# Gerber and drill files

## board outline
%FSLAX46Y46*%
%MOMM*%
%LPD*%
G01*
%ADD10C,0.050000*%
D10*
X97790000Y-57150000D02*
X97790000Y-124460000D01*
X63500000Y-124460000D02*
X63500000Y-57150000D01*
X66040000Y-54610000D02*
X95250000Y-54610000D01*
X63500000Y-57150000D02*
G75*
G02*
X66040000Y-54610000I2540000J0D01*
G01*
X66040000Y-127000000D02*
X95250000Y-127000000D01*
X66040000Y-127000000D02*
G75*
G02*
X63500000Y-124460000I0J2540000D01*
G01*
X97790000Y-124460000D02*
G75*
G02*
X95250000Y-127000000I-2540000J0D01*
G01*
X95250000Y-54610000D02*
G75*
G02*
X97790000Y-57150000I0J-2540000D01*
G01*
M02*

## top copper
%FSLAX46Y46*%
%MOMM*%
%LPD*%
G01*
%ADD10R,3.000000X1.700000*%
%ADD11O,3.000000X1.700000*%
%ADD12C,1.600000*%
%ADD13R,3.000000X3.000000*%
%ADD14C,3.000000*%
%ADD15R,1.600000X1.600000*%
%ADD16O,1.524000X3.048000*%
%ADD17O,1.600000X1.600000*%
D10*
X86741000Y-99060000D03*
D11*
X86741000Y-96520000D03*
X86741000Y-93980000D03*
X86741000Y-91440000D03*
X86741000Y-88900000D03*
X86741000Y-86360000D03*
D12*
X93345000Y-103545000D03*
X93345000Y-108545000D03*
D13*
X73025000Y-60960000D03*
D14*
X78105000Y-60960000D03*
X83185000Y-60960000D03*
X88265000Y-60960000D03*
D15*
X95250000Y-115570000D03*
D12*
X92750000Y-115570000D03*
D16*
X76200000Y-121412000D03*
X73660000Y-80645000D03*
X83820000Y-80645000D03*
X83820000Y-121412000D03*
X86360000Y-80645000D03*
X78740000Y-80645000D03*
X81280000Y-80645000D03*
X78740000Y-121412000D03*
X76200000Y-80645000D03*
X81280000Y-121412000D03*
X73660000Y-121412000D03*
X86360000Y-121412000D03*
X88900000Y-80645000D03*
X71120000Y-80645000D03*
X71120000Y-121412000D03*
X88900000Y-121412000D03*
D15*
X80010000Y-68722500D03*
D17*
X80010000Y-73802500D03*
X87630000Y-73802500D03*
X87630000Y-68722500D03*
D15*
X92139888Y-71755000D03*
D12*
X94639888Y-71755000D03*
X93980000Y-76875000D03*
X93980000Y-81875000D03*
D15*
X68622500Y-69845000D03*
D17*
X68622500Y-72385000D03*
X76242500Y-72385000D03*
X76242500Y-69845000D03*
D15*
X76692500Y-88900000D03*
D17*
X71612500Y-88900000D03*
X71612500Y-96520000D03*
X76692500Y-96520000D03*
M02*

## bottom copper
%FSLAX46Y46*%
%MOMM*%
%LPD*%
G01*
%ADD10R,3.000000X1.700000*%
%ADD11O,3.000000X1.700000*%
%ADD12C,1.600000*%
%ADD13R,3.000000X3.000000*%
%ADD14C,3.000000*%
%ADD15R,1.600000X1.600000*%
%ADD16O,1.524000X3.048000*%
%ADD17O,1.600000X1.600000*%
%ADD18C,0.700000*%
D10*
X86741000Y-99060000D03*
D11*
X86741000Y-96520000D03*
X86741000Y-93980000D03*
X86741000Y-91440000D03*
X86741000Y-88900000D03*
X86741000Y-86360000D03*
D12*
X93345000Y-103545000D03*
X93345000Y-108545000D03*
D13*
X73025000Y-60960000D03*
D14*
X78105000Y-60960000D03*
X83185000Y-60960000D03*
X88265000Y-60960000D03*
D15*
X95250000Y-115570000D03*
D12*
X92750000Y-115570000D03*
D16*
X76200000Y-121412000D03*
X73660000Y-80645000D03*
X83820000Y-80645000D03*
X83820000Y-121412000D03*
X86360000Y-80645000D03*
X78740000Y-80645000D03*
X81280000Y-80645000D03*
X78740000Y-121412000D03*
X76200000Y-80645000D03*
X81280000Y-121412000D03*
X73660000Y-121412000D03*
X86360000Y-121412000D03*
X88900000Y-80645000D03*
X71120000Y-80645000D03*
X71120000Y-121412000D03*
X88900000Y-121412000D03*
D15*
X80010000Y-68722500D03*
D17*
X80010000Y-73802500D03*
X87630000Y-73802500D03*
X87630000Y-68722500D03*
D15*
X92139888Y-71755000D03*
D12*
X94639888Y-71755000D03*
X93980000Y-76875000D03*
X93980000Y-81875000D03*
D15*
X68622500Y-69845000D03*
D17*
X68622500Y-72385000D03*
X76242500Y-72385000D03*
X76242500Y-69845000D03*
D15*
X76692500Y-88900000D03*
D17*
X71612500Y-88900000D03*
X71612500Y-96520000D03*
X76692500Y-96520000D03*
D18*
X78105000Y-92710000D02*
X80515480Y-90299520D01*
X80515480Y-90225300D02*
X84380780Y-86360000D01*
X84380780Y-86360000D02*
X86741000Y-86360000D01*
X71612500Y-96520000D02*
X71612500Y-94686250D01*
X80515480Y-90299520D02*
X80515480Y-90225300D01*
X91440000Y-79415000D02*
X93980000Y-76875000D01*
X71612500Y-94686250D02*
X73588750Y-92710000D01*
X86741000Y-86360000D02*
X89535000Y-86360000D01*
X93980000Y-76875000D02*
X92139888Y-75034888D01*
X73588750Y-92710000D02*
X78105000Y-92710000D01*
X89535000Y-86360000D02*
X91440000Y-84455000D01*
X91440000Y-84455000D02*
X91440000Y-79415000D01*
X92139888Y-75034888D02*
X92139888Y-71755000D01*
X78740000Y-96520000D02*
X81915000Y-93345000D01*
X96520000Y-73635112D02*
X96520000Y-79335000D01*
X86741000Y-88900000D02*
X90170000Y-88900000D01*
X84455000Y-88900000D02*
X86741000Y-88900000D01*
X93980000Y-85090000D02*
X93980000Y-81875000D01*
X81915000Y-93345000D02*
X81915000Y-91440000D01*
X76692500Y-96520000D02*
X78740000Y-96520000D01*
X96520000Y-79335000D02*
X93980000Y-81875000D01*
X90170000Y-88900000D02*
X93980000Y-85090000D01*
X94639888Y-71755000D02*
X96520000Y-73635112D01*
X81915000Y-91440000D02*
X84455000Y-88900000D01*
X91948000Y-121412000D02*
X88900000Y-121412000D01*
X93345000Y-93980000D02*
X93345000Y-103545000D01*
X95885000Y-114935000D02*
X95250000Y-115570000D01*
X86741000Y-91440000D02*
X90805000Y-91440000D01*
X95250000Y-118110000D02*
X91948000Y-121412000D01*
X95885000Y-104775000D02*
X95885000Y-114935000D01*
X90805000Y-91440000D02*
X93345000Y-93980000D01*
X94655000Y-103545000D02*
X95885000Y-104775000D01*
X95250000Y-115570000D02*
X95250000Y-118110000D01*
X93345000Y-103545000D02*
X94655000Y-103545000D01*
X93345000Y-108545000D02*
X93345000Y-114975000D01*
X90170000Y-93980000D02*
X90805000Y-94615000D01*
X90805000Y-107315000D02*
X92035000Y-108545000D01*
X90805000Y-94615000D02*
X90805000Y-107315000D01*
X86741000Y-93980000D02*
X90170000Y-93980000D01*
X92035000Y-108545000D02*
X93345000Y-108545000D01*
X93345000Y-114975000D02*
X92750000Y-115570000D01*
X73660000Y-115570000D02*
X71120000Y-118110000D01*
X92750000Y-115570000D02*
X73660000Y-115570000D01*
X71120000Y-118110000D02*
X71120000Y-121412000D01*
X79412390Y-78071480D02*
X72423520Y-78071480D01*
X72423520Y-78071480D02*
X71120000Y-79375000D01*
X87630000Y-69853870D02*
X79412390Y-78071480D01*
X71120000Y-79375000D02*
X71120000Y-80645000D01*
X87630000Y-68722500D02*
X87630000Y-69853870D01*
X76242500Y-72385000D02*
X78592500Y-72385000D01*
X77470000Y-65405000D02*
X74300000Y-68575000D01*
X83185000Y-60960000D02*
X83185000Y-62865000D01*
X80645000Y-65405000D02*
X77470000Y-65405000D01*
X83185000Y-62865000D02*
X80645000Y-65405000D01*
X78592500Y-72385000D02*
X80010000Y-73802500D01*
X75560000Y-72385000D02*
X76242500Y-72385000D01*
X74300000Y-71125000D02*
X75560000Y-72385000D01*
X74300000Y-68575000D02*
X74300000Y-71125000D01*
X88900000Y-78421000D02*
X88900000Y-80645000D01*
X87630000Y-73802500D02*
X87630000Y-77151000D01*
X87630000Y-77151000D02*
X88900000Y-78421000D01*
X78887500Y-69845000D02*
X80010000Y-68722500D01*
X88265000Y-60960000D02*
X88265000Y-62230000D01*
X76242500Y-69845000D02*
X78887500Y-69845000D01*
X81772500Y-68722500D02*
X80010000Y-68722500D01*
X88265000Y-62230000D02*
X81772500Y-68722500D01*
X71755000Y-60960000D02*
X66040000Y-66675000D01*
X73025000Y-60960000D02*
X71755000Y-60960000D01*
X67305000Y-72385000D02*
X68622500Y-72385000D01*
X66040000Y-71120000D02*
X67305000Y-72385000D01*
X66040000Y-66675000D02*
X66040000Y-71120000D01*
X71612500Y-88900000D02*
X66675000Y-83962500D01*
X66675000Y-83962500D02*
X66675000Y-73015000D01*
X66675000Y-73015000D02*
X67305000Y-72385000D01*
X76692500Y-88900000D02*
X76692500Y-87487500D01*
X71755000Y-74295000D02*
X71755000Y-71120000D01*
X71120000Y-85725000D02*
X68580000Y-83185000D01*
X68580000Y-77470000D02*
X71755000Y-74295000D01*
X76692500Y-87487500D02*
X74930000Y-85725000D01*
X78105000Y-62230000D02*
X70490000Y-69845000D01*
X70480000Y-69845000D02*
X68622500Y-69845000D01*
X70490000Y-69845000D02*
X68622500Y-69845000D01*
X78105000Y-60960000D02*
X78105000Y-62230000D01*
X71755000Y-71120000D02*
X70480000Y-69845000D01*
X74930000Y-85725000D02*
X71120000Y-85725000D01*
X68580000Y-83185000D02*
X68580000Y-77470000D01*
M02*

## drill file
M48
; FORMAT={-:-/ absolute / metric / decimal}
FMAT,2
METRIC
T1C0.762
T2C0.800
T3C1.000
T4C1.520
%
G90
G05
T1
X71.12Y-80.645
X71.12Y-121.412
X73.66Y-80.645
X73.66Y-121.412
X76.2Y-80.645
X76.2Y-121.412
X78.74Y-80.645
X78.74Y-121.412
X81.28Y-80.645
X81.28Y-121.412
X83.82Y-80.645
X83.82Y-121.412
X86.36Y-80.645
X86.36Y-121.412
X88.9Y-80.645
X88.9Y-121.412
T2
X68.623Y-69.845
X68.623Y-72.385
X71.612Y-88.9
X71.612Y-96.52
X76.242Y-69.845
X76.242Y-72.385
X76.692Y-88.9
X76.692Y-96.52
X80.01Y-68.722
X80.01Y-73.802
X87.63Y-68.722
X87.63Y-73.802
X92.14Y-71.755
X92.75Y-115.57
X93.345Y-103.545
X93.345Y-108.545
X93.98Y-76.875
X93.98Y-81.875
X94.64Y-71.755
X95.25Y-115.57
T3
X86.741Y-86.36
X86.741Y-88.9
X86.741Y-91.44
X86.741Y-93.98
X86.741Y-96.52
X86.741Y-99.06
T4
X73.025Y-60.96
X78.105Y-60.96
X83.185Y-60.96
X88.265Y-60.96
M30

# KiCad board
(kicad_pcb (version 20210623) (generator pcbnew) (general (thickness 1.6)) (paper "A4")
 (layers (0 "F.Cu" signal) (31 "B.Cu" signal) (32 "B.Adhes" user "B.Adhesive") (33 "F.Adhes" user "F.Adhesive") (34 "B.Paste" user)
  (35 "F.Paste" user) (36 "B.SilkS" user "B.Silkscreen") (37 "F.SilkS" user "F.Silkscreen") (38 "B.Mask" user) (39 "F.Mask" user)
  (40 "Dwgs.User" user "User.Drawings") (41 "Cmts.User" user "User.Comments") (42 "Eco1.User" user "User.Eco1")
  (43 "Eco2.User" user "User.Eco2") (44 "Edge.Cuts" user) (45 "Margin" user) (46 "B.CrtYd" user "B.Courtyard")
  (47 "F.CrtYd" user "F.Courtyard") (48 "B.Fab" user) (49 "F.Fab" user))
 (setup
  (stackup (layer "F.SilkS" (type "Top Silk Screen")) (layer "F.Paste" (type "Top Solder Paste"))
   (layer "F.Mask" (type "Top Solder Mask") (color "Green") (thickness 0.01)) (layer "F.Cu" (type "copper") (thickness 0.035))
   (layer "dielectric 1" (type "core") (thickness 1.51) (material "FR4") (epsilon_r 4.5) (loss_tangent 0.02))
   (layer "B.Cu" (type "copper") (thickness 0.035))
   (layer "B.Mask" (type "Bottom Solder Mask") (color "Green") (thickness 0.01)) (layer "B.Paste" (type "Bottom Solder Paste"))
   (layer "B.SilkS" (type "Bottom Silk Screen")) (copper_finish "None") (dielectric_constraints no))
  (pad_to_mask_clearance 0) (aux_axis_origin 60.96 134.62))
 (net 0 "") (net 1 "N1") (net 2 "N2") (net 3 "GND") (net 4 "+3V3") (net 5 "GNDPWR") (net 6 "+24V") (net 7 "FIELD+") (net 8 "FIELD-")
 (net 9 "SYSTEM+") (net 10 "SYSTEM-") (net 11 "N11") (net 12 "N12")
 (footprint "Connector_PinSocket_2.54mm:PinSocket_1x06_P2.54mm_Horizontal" (layer "F.Cu") (at 86.741 99.06 180)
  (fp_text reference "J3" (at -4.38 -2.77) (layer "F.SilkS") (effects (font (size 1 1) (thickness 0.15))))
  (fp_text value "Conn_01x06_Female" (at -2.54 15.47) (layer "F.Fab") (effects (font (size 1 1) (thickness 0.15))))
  (pad "1" thru_hole rect locked (at 0 0 180) (size 3 1.7) (drill 1) (layers *.Cu *.Mask) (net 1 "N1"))
  (pad "2" thru_hole oval locked (at 0 2.54 180) (size 3 1.7) (drill 1) (layers *.Cu *.Mask) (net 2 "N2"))
  (pad "3" thru_hole oval locked (at 0 5.08 180) (size 3 1.7) (drill 1) (layers *.Cu *.Mask) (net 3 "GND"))
  (pad "4" thru_hole oval locked (at 0 7.62 180) (size 3 1.7) (drill 1) (layers *.Cu *.Mask) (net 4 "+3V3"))
  (pad "5" thru_hole oval locked (at 0 10.16 180) (size 3 1.7) (drill 1) (layers *.Cu *.Mask) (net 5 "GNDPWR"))
  (pad "6" thru_hole oval locked (at 0 12.7 180) (size 3 1.7) (drill 1) (layers *.Cu *.Mask) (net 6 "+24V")))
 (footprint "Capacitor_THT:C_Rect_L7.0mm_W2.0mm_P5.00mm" (layer "F.Cu") (at 93.345 103.545 -90)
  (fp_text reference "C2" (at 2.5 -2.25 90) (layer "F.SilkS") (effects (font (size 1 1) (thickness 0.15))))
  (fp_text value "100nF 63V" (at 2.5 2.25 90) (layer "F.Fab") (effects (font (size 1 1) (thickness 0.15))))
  (pad "1" thru_hole circle locked (at 0 0 270) (size 1.6 1.6) (drill 0.8) (layers *.Cu *.Mask) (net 4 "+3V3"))
  (pad "2" thru_hole circle locked (at 5 0 270) (size 1.6 1.6) (drill 0.8) (layers *.Cu *.Mask) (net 3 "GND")))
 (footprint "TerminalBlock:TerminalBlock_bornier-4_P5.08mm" (layer "F.Cu") (at 73.025 60.96)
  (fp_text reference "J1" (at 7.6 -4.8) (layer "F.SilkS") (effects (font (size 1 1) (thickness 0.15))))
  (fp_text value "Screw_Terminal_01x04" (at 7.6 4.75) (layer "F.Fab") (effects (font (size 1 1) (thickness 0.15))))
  (pad "1" thru_hole rect locked (at 0 0) (size 3 3) (drill 1.52) (layers *.Cu *.Mask) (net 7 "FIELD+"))
  (pad "2" thru_hole circle locked (at 5.08 0) (size 3 3) (drill 1.52) (layers *.Cu *.Mask) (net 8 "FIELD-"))
  (pad "3" thru_hole circle locked (at 10.16 0) (size 3 3) (drill 1.52) (layers *.Cu *.Mask) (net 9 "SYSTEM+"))
  (pad "4" thru_hole circle locked (at 15.24 0) (size 3 3) (drill 1.52) (layers *.Cu *.Mask) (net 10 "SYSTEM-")))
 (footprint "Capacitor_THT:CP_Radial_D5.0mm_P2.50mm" (layer "F.Cu") (at 95.25 115.57 180)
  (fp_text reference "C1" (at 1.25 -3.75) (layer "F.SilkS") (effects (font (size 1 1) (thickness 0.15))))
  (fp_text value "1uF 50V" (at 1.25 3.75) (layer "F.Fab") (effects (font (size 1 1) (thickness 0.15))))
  (pad "1" thru_hole rect locked (at 0 0 180) (size 1.6 1.6) (drill 0.8) (layers *.Cu *.Mask) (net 4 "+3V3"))
  (pad "2" thru_hole circle locked (at 2.5 0 180) (size 1.6 1.6) (drill 0.8) (layers *.Cu *.Mask) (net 3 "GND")))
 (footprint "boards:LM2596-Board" (layer "F.Cu") (at 80.01 100.965 -90)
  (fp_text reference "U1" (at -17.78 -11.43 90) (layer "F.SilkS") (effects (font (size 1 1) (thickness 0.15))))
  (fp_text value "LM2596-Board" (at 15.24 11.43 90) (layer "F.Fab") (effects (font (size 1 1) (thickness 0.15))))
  (pad "" thru_hole oval locked (at 20.447 3.81 270) (size 3.048 1.524) (drill 0.762) (layers *.Cu *.Mask))
  (pad "" thru_hole oval locked (at -20.32 6.35 270) (size 3.048 1.524) (drill 0.762) (layers *.Cu *.Mask))
  (pad "" thru_hole oval locked (at -20.32 -3.81 270) (size 3.048 1.524) (drill 0.762) (layers *.Cu *.Mask))
  (pad "" thru_hole oval locked (at 20.447 -3.81 270) (size 3.048 1.524) (drill 0.762) (layers *.Cu *.Mask))
  (pad "" thru_hole oval locked (at -20.32 -6.35 270) (size 3.048 1.524) (drill 0.762) (layers *.Cu *.Mask))
  (pad "" thru_hole oval locked (at -20.32 1.27 270) (size 3.048 1.524) (drill 0.762) (layers *.Cu *.Mask))
  (pad "" thru_hole oval locked (at -20.32 -1.27 270) (size 3.048 1.524) (drill 0.762) (layers *.Cu *.Mask))
  (pad "" thru_hole oval locked (at 20.447 1.27 270) (size 3.048 1.524) (drill 0.762) (layers *.Cu *.Mask))
  (pad "" thru_hole oval locked (at -20.32 3.81 270) (size 3.048 1.524) (drill 0.762) (layers *.Cu *.Mask))
  (pad "" thru_hole oval locked (at 20.447 -1.27 270) (size 3.048 1.524) (drill 0.762) (layers *.Cu *.Mask))
  (pad "" thru_hole oval locked (at 20.447 6.35 270) (size 3.048 1.524) (drill 0.762) (layers *.Cu *.Mask))
  (pad "" thru_hole oval locked (at 20.447 -6.35 270) (size 3.048 1.524) (drill 0.762) (layers *.Cu *.Mask))
  (pad "1" thru_hole oval locked (at -20.32 -8.89 270) (size 3.048 1.524) (drill 0.762) (layers *.Cu *.Mask) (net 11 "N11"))
  (pad "2" thru_hole oval locked (at -20.32 8.89 270) (size 3.048 1.524) (drill 0.762) (layers *.Cu *.Mask) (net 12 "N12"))
  (pad "3" thru_hole oval locked (at 20.447 8.89 270) (size 3.048 1.524) (drill 0.762) (layers *.Cu *.Mask) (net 3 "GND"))
  (pad "4" thru_hole oval locked (at 20.447 -8.89 270) (size 3.048 1.524) (drill 0.762) (layers *.Cu *.Mask) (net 4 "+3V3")))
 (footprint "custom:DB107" (layer "F.Cu") (at 80.01 68.7225)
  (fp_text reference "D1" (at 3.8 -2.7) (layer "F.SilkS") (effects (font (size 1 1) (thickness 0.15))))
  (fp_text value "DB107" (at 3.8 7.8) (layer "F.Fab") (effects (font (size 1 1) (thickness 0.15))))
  (pad "1" thru_hole rect locked (at 0 0) (size 1.6 1.6) (drill 0.8) (layers *.Cu *.Mask) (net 10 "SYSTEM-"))
  (pad "2" thru_hole oval locked (at 0 5.08) (size 1.6 1.6) (drill 0.8) (layers *.Cu *.Mask) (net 9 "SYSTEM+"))
  (pad "3" thru_hole oval locked (at 7.62 5.08) (size 1.6 1.6) (drill 0.8) (layers *.Cu *.Mask) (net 11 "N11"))
  (pad "4" thru_hole oval locked (at 7.62 0) (size 1.6 1.6) (drill 0.8) (layers *.Cu *.Mask) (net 12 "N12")))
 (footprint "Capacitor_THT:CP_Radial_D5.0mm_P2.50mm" (layer "F.Cu") (at 92.139888 71.755)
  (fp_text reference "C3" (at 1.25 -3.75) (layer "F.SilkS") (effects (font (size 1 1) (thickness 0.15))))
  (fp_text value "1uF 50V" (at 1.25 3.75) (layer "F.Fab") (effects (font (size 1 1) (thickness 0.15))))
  (pad "1" thru_hole rect locked (at 0 0) (size 1.6 1.6) (drill 0.8) (layers *.Cu *.Mask) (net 6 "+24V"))
  (pad "2" thru_hole circle locked (at 2.5 0) (size 1.6 1.6) (drill 0.8) (layers *.Cu *.Mask) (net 5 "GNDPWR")))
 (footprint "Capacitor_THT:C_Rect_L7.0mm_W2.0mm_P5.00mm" (layer "F.Cu") (at 93.98 76.875 -90)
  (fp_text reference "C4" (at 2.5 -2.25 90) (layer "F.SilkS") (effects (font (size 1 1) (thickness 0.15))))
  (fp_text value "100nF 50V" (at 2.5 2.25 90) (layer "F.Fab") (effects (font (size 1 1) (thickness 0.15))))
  (pad "1" thru_hole circle locked (at 0 0 270) (size 1.6 1.6) (drill 0.8) (layers *.Cu *.Mask) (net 6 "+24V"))
  (pad "2" thru_hole circle locked (at 5 0 270) (size 1.6 1.6) (drill 0.8) (layers *.Cu *.Mask) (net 5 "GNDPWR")))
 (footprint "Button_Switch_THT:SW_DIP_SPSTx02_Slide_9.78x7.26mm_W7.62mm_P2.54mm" (layer "F.Cu") (at 68.6225 69.845)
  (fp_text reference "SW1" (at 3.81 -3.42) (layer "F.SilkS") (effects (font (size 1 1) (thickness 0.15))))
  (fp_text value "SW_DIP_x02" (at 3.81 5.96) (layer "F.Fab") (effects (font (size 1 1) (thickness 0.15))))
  (pad "1" thru_hole rect locked (at 0 0) (size 1.6 1.6) (drill 0.8) (layers *.Cu *.Mask) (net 8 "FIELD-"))
  (pad "2" thru_hole oval locked (at 0 2.54) (size 1.6 1.6) (drill 0.8) (layers *.Cu *.Mask) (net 7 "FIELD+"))
  (pad "3" thru_hole oval locked (at 7.62 2.54) (size 1.6 1.6) (drill 0.8) (layers *.Cu *.Mask) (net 9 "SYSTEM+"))
  (pad "4" thru_hole oval locked (at 7.62 0) (size 1.6 1.6) (drill 0.8) (layers *.Cu *.Mask) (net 10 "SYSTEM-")))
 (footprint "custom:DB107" (layer "F.Cu") (at 76.6925 88.9 -90)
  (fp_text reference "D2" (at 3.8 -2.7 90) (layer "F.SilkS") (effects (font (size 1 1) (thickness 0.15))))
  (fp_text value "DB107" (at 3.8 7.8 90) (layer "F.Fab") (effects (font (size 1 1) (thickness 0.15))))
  (pad "1" thru_hole rect locked (at 0 0 270) (size 1.6 1.6) (drill 0.8) (layers *.Cu *.Mask) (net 8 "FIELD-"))
  (pad "2" thru_hole oval locked (at 0 5.08 270) (size 1.6 1.6) (drill 0.8) (layers *.Cu *.Mask) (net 7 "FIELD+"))
  (pad "3" thru_hole oval locked (at 7.62 5.08 270) (size 1.6 1.6) (drill 0.8) (layers *.Cu *.Mask) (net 6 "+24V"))
  (pad "4" thru_hole oval locked (at 7.62 0 270) (size 1.6 1.6) (drill 0.8) (layers *.Cu *.Mask) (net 5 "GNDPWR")))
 (gr_line (start 97.79 57.15) (end 97.79 124.46) (layer "Edge.Cuts") (width 0.05))
 (gr_line (start 63.5 124.46) (end 63.5 57.15) (layer "Edge.Cuts") (width 0.05))
 (gr_line (start 66.04 54.61) (end 95.25 54.61) (layer "Edge.Cuts") (width 0.05))
 (gr_arc (start 66.04 57.15) (end 66.04 54.61) (angle -90) (layer "Edge.Cuts") (width 0.05))
 (gr_line (start 66.04 127) (end 95.25 127) (layer "Edge.Cuts") (width 0.05))
 (gr_arc (start 66.04 124.46) (end 63.5 124.46) (angle -90) (layer "Edge.Cuts") (width 0.05))
 (gr_arc (start 95.25 124.46) (end 95.25 127) (angle -90) (layer "Edge.Cuts") (width 0.05))
 (gr_arc (start 95.25 57.15) (end 97.79 57.15) (angle -90) (layer "Edge.Cuts") (width 0.05))
 (segment (start 78.105 92.71) (end 80.51548 90.29952) (width 0.7) (layer "B.Cu") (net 6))
 (segment (start 80.51548 90.2253) (end 84.38078 86.36) (width 0.7) (layer "B.Cu") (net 6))
 (segment (start 84.38078 86.36) (end 86.741 86.36) (width 0.7) (layer "B.Cu") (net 6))
 (segment (start 71.6125 96.52) (end 71.6125 94.68625) (width 0.7) (layer "B.Cu") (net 6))
 (segment (start 80.51548 90.29952) (end 80.51548 90.2253) (width 0.7) (layer "B.Cu") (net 6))
 (segment (start 91.44 79.415) (end 93.98 76.875) (width 0.7) (layer "B.Cu") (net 6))
 (segment (start 71.6125 94.68625) (end 73.58875 92.71) (width 0.7) (layer "B.Cu") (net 6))
 (segment (start 86.741 86.36) (end 89.535 86.36) (width 0.7) (layer "B.Cu") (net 6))
 (segment (start 93.98 76.875) (end 92.139888 75.034888) (width 0.7) (layer "B.Cu") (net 6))
 (segment (start 73.58875 92.71) (end 78.105 92.71) (width 0.7) (layer "B.Cu") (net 6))
 (segment (start 89.535 86.36) (end 91.44 84.455) (width 0.7) (layer "B.Cu") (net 6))
 (segment (start 91.44 84.455) (end 91.44 79.415) (width 0.7) (layer "B.Cu") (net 6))
 (segment (start 92.139888 75.034888) (end 92.139888 71.755) (width 0.7) (layer "B.Cu") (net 6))
 (segment (start 78.74 96.52) (end 81.915 93.345) (width 0.7) (layer "B.Cu") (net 5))
 (segment (start 96.52 73.635112) (end 96.52 79.335) (width 0.7) (layer "B.Cu") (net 5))
 (segment (start 86.741 88.9) (end 90.17 88.9) (width 0.7) (layer "B.Cu") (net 5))
 (segment (start 84.455 88.9) (end 86.741 88.9) (width 0.7) (layer "B.Cu") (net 5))
 (segment (start 93.98 85.09) (end 93.98 81.875) (width 0.7) (layer "B.Cu") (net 5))
 (segment (start 81.915 93.345) (end 81.915 91.44) (width 0.7) (layer "B.Cu") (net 5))
 (segment (start 76.6925 96.52) (end 78.74 96.52) (width 0.7) (layer "B.Cu") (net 5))
 (segment (start 96.52 79.335) (end 93.98 81.875) (width 0.7) (layer "B.Cu") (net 5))
 (segment (start 90.17 88.9) (end 93.98 85.09) (width 0.7) (layer "B.Cu") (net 5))
 (segment (start 94.639888 71.755) (end 96.52 73.635112) (width 0.7) (layer "B.Cu") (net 5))
 (segment (start 81.915 91.44) (end 84.455 88.9) (width 0.7) (layer "B.Cu") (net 5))
 (segment (start 91.948 121.412) (end 88.9 121.412) (width 0.7) (layer "B.Cu") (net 4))
 (segment (start 93.345 93.98) (end 93.345 103.545) (width 0.7) (layer "B.Cu") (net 4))
 (segment (start 95.885 114.935) (end 95.25 115.57) (width 0.7) (layer "B.Cu") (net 4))
 (segment (start 86.741 91.44) (end 90.805 91.44) (width 0.7) (layer "B.Cu") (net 4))
 (segment (start 95.25 118.11) (end 91.948 121.412) (width 0.7) (layer "B.Cu") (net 4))
 (segment (start 95.885 104.775) (end 95.885 114.935) (width 0.7) (layer "B.Cu") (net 4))
 (segment (start 90.805 91.44) (end 93.345 93.98) (width 0.7) (layer "B.Cu") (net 4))
 (segment (start 94.655 103.545) (end 95.885 104.775) (width 0.7) (layer "B.Cu") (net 4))
 (segment (start 95.25 115.57) (end 95.25 118.11) (width 0.7) (layer "B.Cu") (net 4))
 (segment (start 93.345 103.545) (end 94.655 103.545) (width 0.7) (layer "B.Cu") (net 4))
 (segment (start 93.345 108.545) (end 93.345 114.975) (width 0.7) (layer "B.Cu") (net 3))
 (segment (start 90.17 93.98) (end 90.805 94.615) (width 0.7) (layer "B.Cu") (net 3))
 (segment (start 90.805 107.315) (end 92.035 108.545) (width 0.7) (layer "B.Cu") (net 3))
 (segment (start 90.805 94.615) (end 90.805 107.315) (width 0.7) (layer "B.Cu") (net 3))
 (segment (start 86.741 93.98) (end 90.17 93.98) (width 0.7) (layer "B.Cu") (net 3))
 (segment (start 92.035 108.545) (end 93.345 108.545) (width 0.7) (layer "B.Cu") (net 3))
 (segment (start 93.345 114.975) (end 92.75 115.57) (width 0.7) (layer "B.Cu") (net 3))
 (segment (start 73.66 115.57) (end 71.12 118.11) (width 0.7) (layer "B.Cu") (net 3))
 (segment (start 92.75 115.57) (end 73.66 115.57) (width 0.7) (layer "B.Cu") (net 3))
 (segment (start 71.12 118.11) (end 71.12 121.412) (width 0.7) (layer "B.Cu") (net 3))
 (segment (start 79.41239 78.07148) (end 72.42352 78.07148) (width 0.7) (layer "B.Cu") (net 12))
 (segment (start 72.42352 78.07148) (end 71.12 79.375) (width 0.7) (layer "B.Cu") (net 12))
 (segment (start 87.63 69.85387) (end 79.41239 78.07148) (width 0.7) (layer "B.Cu") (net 12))
 (segment (start 71.12 79.375) (end 71.12 80.645) (width 0.7) (layer "B.Cu") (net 12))
 (segment (start 87.63 68.7225) (end 87.63 69.85387) (width 0.7) (layer "B.Cu") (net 12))
 (segment (start 76.2425 72.385) (end 78.5925 72.385) (width 0.7) (layer "B.Cu") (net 9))
 (segment (start 77.47 65.405) (end 74.3 68.575) (width 0.7) (layer "B.Cu") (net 9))
 (segment (start 83.185 60.96) (end 83.185 62.865) (width 0.7) (layer "B.Cu") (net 9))
 (segment (start 80.645 65.405) (end 77.47 65.405) (width 0.7) (layer "B.Cu") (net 9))
 (segment (start 83.185 62.865) (end 80.645 65.405) (width 0.7) (layer "B.Cu") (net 9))
 (segment (start 78.5925 72.385) (end 80.01 73.8025) (width 0.7) (layer "B.Cu") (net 9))
 (segment (start 75.56 72.385) (end 76.2425 72.385) (width 0.7) (layer "B.Cu") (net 9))
 (segment (start 74.3 71.125) (end 75.56 72.385) (width 0.7) (layer "B.Cu") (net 9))
 (segment (start 74.3 68.575) (end 74.3 71.125) (width 0.7) (layer "B.Cu") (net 9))
 (segment (start 88.9 78.421) (end 88.9 80.645) (width 0.7) (layer "B.Cu") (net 11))
 (segment (start 87.63 73.8025) (end 87.63 77.151) (width 0.7) (layer "B.Cu") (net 11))
 (segment (start 87.63 77.151) (end 88.9 78.421) (width 0.7) (layer "B.Cu") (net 11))
 (segment (start 78.8875 69.845) (end 80.01 68.7225) (width 0.7) (layer "B.Cu") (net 10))
 (segment (start 88.265 60.96) (end 88.265 62.23) (width 0.7) (layer "B.Cu") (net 10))
 (segment (start 76.2425 69.845) (end 78.8875 69.845) (width 0.7) (layer "B.Cu") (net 10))
 (segment (start 81.7725 68.7225) (end 80.01 68.7225) (width 0.7) (layer "B.Cu") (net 10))
 (segment (start 88.265 62.23) (end 81.7725 68.7225) (width 0.7) (layer "B.Cu") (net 10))
 (segment (start 71.755 60.96) (end 66.04 66.675) (width 0.7) (layer "B.Cu") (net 7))
 (segment (start 73.025 60.96) (end 71.755 60.96) (width 0.7) (layer "B.Cu") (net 7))
 (segment (start 67.305 72.385) (end 68.6225 72.385) (width 0.7) (layer "B.Cu") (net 7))
 (segment (start 66.04 71.12) (end 67.305 72.385) (width 0.7) (layer "B.Cu") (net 7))
 (segment (start 66.04 66.675) (end 66.04 71.12) (width 0.7) (layer "B.Cu") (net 7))
 (segment (start 71.6125 88.9) (end 66.675 83.9625) (width 0.7) (layer "B.Cu") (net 7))
 (segment (start 66.675 83.9625) (end 66.675 73.015) (width 0.7) (layer "B.Cu") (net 7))
 (segment (start 66.675 73.015) (end 67.305 72.385) (width 0.7) (layer "B.Cu") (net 7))
 (segment (start 76.6925 88.9) (end 76.6925 87.4875) (width 0.7) (layer "B.Cu") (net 8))
 (segment (start 71.755 74.295) (end 71.755 71.12) (width 0.7) (layer "B.Cu") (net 8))
 (segment (start 71.12 85.725) (end 68.58 83.185) (width 0.7) (layer "B.Cu") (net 8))
 (segment (start 68.58 77.47) (end 71.755 74.295) (width 0.7) (layer "B.Cu") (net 8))
 (segment (start 76.6925 87.4875) (end 74.93 85.725) (width 0.7) (layer "B.Cu") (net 8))
 (segment (start 78.105 62.23) (end 70.49 69.845) (width 0.7) (layer "B.Cu") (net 8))
 (segment (start 70.48 69.845) (end 68.6225 69.845) (width 0.7) (layer "B.Cu") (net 8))
 (segment (start 70.49 69.845) (end 68.6225 69.845) (width 0.7) (layer "B.Cu") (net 8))
 (segment (start 78.105 60.96) (end 78.105 62.23) (width 0.7) (layer "B.Cu") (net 8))
 (segment (start 71.755 71.12) (end 70.48 69.845) (width 0.7) (layer "B.Cu") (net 8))
 (segment (start 74.93 85.725) (end 71.12 85.725) (width 0.7) (layer "B.Cu") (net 8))
 (segment (start 68.58 83.185) (end 68.58 77.47) (width 0.7) (layer "B.Cu") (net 8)))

